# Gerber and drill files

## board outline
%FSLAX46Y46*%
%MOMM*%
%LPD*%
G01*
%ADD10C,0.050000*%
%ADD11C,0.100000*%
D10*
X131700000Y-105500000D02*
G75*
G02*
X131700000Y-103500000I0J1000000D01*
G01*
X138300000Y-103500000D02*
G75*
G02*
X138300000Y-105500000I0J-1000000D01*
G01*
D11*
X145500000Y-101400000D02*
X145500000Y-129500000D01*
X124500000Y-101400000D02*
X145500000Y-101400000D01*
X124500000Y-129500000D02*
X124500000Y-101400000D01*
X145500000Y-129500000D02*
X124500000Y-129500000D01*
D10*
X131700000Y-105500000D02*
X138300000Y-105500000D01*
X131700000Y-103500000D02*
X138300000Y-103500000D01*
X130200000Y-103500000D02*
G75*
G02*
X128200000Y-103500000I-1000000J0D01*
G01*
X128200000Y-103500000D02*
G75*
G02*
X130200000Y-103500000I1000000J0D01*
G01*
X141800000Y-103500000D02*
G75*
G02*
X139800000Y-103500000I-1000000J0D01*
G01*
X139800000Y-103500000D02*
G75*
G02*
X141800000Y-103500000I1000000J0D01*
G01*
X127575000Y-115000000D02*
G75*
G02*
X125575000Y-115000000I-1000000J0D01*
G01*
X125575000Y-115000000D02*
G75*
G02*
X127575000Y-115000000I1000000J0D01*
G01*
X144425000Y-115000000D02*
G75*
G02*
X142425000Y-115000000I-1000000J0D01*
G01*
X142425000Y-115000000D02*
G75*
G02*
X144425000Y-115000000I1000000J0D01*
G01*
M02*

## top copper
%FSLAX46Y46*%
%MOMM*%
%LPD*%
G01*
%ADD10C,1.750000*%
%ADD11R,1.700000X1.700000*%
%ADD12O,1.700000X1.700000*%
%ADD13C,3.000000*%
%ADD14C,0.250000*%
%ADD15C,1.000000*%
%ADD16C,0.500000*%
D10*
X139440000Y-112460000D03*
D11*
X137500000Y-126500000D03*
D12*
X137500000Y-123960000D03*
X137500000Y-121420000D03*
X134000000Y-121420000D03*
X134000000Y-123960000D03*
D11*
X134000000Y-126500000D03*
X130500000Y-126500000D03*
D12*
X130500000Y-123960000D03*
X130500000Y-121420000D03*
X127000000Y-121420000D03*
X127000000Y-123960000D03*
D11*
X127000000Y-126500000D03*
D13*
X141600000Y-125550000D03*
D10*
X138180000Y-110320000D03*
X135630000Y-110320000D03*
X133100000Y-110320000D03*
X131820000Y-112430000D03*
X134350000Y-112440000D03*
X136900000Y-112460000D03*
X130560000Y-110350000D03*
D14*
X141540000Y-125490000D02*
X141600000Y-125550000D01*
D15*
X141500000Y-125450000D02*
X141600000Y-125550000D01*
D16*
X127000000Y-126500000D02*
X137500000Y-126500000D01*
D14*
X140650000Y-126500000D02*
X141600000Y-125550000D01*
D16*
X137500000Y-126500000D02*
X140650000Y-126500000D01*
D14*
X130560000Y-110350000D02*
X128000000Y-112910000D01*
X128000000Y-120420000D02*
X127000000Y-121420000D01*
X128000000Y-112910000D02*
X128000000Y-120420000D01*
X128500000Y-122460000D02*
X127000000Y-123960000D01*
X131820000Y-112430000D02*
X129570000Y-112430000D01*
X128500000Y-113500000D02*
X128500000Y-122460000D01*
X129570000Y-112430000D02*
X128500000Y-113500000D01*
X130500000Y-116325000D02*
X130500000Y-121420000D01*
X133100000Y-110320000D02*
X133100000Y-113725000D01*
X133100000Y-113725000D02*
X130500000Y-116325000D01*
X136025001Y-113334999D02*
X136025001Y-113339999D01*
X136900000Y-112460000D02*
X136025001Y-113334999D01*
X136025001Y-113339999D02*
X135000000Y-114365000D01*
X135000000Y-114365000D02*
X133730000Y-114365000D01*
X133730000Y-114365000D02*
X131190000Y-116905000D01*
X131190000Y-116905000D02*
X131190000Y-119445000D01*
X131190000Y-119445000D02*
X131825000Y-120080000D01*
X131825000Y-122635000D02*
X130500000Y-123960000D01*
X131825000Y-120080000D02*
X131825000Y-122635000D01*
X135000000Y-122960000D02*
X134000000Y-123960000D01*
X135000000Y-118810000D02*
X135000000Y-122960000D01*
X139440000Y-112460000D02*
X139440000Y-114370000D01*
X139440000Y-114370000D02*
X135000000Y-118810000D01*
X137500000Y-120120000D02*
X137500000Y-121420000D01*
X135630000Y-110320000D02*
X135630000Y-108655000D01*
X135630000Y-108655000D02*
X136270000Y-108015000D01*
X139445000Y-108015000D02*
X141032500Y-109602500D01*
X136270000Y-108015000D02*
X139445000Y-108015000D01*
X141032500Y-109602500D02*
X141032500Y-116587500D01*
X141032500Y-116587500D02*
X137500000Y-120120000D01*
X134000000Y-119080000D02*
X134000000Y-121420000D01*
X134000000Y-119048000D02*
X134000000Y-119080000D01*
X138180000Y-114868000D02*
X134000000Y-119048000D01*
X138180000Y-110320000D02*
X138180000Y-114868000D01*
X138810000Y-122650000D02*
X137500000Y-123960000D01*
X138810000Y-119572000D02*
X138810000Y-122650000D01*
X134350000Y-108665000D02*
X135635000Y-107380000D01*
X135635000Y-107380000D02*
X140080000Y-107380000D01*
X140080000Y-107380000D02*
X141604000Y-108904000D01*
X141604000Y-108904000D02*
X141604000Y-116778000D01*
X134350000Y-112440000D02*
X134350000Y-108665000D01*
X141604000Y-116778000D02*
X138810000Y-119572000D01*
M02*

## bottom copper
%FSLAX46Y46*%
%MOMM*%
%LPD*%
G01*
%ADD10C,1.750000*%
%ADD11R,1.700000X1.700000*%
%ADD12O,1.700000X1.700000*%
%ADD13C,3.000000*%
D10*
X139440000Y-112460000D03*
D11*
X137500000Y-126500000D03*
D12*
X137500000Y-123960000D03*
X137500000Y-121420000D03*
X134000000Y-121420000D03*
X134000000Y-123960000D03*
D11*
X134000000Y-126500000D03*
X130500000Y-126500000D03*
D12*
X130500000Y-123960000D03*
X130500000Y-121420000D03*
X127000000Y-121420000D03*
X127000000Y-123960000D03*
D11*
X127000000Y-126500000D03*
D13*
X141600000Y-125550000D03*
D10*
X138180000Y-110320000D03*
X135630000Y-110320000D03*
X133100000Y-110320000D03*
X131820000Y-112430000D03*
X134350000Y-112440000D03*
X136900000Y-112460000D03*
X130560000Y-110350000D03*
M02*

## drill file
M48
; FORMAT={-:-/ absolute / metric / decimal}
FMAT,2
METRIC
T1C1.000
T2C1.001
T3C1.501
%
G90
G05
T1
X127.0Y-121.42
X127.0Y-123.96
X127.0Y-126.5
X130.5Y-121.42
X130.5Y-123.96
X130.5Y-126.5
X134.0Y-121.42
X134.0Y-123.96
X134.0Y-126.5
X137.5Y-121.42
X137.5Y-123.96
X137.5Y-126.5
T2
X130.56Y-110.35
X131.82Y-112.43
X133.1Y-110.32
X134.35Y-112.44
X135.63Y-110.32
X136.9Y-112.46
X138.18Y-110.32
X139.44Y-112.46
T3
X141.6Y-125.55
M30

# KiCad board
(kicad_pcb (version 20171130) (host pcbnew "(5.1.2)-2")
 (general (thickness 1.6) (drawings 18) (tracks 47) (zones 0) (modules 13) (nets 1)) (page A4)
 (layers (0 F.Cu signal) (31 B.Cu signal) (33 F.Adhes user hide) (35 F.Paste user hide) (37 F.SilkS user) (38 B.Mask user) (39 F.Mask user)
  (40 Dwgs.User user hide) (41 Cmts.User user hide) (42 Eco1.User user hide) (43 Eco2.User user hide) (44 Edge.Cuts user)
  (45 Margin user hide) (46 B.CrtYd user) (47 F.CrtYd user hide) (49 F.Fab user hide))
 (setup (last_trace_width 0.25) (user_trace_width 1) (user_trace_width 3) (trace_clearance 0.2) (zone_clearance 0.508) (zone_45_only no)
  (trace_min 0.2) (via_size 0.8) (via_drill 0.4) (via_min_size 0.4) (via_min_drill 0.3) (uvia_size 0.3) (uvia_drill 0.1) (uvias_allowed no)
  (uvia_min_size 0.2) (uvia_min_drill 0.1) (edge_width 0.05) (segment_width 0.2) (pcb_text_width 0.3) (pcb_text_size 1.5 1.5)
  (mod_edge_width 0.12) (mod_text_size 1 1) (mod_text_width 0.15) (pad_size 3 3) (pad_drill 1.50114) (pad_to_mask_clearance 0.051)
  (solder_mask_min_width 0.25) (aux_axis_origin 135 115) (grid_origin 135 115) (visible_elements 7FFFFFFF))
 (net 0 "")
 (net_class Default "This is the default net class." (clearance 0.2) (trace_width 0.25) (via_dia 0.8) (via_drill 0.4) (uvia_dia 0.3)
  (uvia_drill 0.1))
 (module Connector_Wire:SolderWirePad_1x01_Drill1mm (layer F.Cu) (at 139.44 112.46)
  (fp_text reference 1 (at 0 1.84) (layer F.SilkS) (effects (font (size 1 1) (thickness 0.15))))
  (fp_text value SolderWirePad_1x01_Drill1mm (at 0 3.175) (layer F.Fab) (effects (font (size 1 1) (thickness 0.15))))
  (pad 1 thru_hole circle (at 0 0) (size 1.75 1.75) (drill 1.00076) (layers *.Cu *.Mask)))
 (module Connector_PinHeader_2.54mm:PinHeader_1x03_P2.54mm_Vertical (layer F.Cu) (at 137.5 126.5 180)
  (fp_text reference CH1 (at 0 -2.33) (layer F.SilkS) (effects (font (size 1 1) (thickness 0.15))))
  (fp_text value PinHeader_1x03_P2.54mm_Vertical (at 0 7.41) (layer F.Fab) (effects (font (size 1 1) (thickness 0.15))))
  (pad 1 thru_hole rect (at 0 0 180) (size 1.7 1.7) (drill 1) (layers *.Cu *.Mask))
  (pad 2 thru_hole oval (at 0 2.54 180) (size 1.7 1.7) (drill 1) (layers *.Cu *.Mask))
  (pad 3 thru_hole oval (at 0 5.08 180) (size 1.7 1.7) (drill 1) (layers *.Cu *.Mask)))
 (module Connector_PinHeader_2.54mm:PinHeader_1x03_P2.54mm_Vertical (layer F.Cu) (at 134 126.5 180)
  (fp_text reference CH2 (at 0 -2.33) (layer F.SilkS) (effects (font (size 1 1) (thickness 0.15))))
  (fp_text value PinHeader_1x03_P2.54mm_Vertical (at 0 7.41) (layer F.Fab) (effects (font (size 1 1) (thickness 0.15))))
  (pad 3 thru_hole oval (at 0 5.08 180) (size 1.7 1.7) (drill 1) (layers *.Cu *.Mask))
  (pad 2 thru_hole oval (at 0 2.54 180) (size 1.7 1.7) (drill 1) (layers *.Cu *.Mask))
  (pad 1 thru_hole rect (at 0 0 180) (size 1.7 1.7) (drill 1) (layers *.Cu *.Mask)))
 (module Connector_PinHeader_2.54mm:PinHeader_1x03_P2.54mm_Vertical (layer F.Cu) (at 130.5 126.5 180)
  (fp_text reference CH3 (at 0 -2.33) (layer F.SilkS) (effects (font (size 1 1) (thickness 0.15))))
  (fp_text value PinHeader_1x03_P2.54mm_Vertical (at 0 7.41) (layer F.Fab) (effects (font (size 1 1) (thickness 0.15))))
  (pad 1 thru_hole rect (at 0 0 180) (size 1.7 1.7) (drill 1) (layers *.Cu *.Mask))
  (pad 2 thru_hole oval (at 0 2.54 180) (size 1.7 1.7) (drill 1) (layers *.Cu *.Mask))
  (pad 3 thru_hole oval (at 0 5.08 180) (size 1.7 1.7) (drill 1) (layers *.Cu *.Mask)))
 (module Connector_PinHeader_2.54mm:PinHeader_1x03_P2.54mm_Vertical (layer F.Cu) (at 127 126.5 180)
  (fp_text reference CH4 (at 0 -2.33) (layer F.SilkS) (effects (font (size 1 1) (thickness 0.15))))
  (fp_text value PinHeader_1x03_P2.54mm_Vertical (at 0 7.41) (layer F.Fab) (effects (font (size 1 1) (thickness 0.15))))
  (pad 3 thru_hole oval (at 0 5.08 180) (size 1.7 1.7) (drill 1) (layers *.Cu *.Mask))
  (pad 2 thru_hole oval (at 0 2.54 180) (size 1.7 1.7) (drill 1) (layers *.Cu *.Mask))
  (pad 1 thru_hole rect (at 0 0 180) (size 1.7 1.7) (drill 1) (layers *.Cu *.Mask)))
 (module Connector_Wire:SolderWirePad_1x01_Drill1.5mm (layer F.Cu) (at 141.6 125.55)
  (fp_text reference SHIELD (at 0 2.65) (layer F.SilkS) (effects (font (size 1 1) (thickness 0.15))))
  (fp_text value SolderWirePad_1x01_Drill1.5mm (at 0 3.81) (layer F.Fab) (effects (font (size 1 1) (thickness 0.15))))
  (pad 1 thru_hole circle (at 0 0) (size 3 3) (drill 1.50114) (layers *.Cu *.Mask)))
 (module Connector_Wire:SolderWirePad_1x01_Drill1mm (layer F.Cu) (at 138.18 110.32)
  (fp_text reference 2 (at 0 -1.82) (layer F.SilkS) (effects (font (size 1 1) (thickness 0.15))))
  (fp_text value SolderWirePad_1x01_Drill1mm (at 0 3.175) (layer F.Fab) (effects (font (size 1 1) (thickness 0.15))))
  (pad 1 thru_hole circle (at 0 0) (size 1.75 1.75) (drill 1.00076) (layers *.Cu *.Mask)))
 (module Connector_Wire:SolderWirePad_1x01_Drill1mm (layer F.Cu) (at 135.63 110.32)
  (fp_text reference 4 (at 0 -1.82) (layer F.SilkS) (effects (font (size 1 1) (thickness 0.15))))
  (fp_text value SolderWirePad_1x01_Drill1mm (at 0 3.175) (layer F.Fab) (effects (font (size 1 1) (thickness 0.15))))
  (pad 1 thru_hole circle (at 0 0) (size 1.75 1.75) (drill 1.00076) (layers *.Cu *.Mask)))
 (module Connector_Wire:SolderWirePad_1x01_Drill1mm (layer F.Cu) (at 133.1 110.32)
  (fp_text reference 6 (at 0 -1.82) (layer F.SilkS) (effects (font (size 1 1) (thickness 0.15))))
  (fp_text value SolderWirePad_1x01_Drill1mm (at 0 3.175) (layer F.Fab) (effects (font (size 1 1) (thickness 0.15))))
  (pad 1 thru_hole circle (at 0 0) (size 1.75 1.75) (drill 1.00076) (layers *.Cu *.Mask)))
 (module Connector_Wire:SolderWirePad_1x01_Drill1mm (layer F.Cu) (at 131.82 112.43)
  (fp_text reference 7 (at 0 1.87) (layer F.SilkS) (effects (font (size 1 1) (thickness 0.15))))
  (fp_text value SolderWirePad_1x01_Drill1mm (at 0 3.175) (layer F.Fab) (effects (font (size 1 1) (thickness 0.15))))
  (pad 1 thru_hole circle (at 0 0) (size 1.75 1.75) (drill 1.00076) (layers *.Cu *.Mask)))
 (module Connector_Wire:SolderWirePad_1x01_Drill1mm (layer F.Cu) (at 134.35 112.44)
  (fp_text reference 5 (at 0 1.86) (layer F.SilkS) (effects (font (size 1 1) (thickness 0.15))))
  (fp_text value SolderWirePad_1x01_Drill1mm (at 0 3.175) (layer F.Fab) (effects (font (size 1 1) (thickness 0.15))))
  (pad 1 thru_hole circle (at 0 0) (size 1.75 1.75) (drill 1.00076) (layers *.Cu *.Mask)))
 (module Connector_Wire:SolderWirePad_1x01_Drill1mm (layer F.Cu) (at 136.9 112.46)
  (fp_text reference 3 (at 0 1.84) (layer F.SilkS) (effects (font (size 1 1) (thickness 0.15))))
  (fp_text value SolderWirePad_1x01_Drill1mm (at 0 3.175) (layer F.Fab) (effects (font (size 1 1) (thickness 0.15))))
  (pad 1 thru_hole circle (at 0 0) (size 1.75 1.75) (drill 1.00076) (layers *.Cu *.Mask)))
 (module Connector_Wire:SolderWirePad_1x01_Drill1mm (layer F.Cu) (at 130.56 110.35)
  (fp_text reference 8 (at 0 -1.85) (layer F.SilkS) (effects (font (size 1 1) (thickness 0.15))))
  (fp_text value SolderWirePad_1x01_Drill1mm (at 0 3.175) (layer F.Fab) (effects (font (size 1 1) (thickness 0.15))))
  (pad 1 thru_hole circle (at 0 0) (size 1.75 1.75) (drill 1.00076) (layers *.Cu *.Mask)))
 (gr_arc (start 131.7 104.5) (end 131.7 103.5) (angle -180) (layer Edge.Cuts) (width 0.05))
 (gr_arc (start 138.3 104.5) (end 138.3 105.5) (angle -180) (layer Edge.Cuts) (width 0.05))
 (gr_line (start 145.5 101.4) (end 145.5 129.5) (layer Edge.Cuts) (width 0.1))
 (gr_line (start 124.5 101.4) (end 145.5 101.4) (layer Edge.Cuts) (width 0.1))
 (gr_line (start 124.5 129.5) (end 124.5 101.4) (layer Edge.Cuts) (width 0.1))
 (gr_line (start 145.5 129.5) (end 124.5 129.5) (layer Edge.Cuts) (width 0.1))
 (gr_line (start 131.7 105.5) (end 138.3 105.5) (layer Edge.Cuts) (width 0.05))
 (gr_line (start 131.7 103.5) (end 138.3 103.5) (layer Edge.Cuts) (width 0.05))
 (gr_circle (center 129.2 103.5) (end 130.2 103.5) (layer Edge.Cuts) (width 0.05))
 (gr_circle (center 140.8 103.5) (end 141.8 103.5) (layer Edge.Cuts) (width 0.05))
 (gr_circle (center 126.575 115) (end 127.575 115) (layer Edge.Cuts) (width 0.05))
 (gr_circle (center 143.425 115) (end 144.425 115) (layer Edge.Cuts) (width 0.05))
 (segment (start 141.54 125.49) (end 141.6 125.55) (width 0.25) (layer F.Cu) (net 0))
 (segment (start 141.5 125.45) (end 141.6 125.55) (width 1) (layer F.Cu) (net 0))
 (segment (start 127 126.5) (end 137.5 126.5) (width 0.5) (layer F.Cu) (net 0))
 (segment (start 140.65 126.5) (end 141.6 125.55) (width 0.25) (layer F.Cu) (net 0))
 (segment (start 137.5 126.5) (end 140.65 126.5) (width 0.5) (layer F.Cu) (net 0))
 (segment (start 130.56 110.35) (end 128 112.91) (width 0.25) (layer F.Cu) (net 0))
 (segment (start 128 120.42) (end 127 121.42) (width 0.25) (layer F.Cu) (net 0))
 (segment (start 128 112.91) (end 128 120.42) (width 0.25) (layer F.Cu) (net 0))
 (segment (start 128.5 122.46) (end 127 123.96) (width 0.25) (layer F.Cu) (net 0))
 (segment (start 131.82 112.43) (end 129.57 112.43) (width 0.25) (layer F.Cu) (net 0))
 (segment (start 128.5 113.5) (end 128.5 122.46) (width 0.25) (layer F.Cu) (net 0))
 (segment (start 129.57 112.43) (end 128.5 113.5) (width 0.25) (layer F.Cu) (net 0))
 (segment (start 130.5 116.325) (end 130.5 121.42) (width 0.25) (layer F.Cu) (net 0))
 (segment (start 133.1 110.32) (end 133.1 113.725) (width 0.25) (layer F.Cu) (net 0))
 (segment (start 133.1 113.725) (end 130.5 116.325) (width 0.25) (layer F.Cu) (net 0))
 (segment (start 136.025001 113.334999) (end 136.025001 113.339999) (width 0.25) (layer F.Cu) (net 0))
 (segment (start 136.9 112.46) (end 136.025001 113.334999) (width 0.25) (layer F.Cu) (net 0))
 (segment (start 136.025001 113.339999) (end 135 114.365) (width 0.25) (layer F.Cu) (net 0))
 (segment (start 135 114.365) (end 133.73 114.365) (width 0.25) (layer F.Cu) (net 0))
 (segment (start 133.73 114.365) (end 131.19 116.905) (width 0.25) (layer F.Cu) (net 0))
 (segment (start 131.19 116.905) (end 131.19 119.445) (width 0.25) (layer F.Cu) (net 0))
 (segment (start 131.19 119.445) (end 131.825 120.08) (width 0.25) (layer F.Cu) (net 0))
 (segment (start 131.825 122.635) (end 130.5 123.96) (width 0.25) (layer F.Cu) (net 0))
 (segment (start 131.825 120.08) (end 131.825 122.635) (width 0.25) (layer F.Cu) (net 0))
 (segment (start 135 122.96) (end 134 123.96) (width 0.25) (layer F.Cu) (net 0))
 (segment (start 135 118.81) (end 135 122.96) (width 0.25) (layer F.Cu) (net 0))
 (segment (start 139.44 112.46) (end 139.44 114.37) (width 0.25) (layer F.Cu) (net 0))
 (segment (start 139.44 114.37) (end 135 118.81) (width 0.25) (layer F.Cu) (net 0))
 (segment (start 137.5 120.12) (end 137.5 121.42) (width 0.25) (layer F.Cu) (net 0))
 (segment (start 135.63 110.32) (end 135.63 108.655) (width 0.25) (layer F.Cu) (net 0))
 (segment (start 135.63 108.655) (end 136.27 108.015) (width 0.25) (layer F.Cu) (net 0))
 (segment (start 139.445 108.015) (end 141.0325 109.6025) (width 0.25) (layer F.Cu) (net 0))
 (segment (start 136.27 108.015) (end 139.445 108.015) (width 0.25) (layer F.Cu) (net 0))
 (segment (start 141.0325 109.6025) (end 141.0325 116.5875) (width 0.25) (layer F.Cu) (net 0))
 (segment (start 141.0325 116.5875) (end 137.5 120.12) (width 0.25) (layer F.Cu) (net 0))
 (segment (start 134 119.08) (end 134 121.42) (width 0.25) (layer F.Cu) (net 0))
 (segment (start 134 119.048) (end 134 119.08) (width 0.25) (layer F.Cu) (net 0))
 (segment (start 138.18 114.868) (end 134 119.048) (width 0.25) (layer F.Cu) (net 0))
 (segment (start 138.18 110.32) (end 138.18 114.868) (width 0.25) (layer F.Cu) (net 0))
 (segment (start 138.81 122.65) (end 137.5 123.96) (width 0.25) (layer F.Cu) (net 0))
 (segment (start 138.81 119.572) (end 138.81 122.65) (width 0.25) (layer F.Cu) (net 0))
 (segment (start 134.35 108.665) (end 135.635 107.38) (width 0.25) (layer F.Cu) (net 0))
 (segment (start 135.635 107.38) (end 140.08 107.38) (width 0.25) (layer F.Cu) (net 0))
 (segment (start 140.08 107.38) (end 141.604 108.904) (width 0.25) (layer F.Cu) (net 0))
 (segment (start 141.604 108.904) (end 141.604 116.778) (width 0.25) (layer F.Cu) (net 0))
 (segment (start 134.35 112.44) (end 134.35 108.665) (width 0.25) (layer F.Cu) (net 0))
 (segment (start 141.604 116.778) (end 138.81 119.572) (width 0.25) (layer F.Cu) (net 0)))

